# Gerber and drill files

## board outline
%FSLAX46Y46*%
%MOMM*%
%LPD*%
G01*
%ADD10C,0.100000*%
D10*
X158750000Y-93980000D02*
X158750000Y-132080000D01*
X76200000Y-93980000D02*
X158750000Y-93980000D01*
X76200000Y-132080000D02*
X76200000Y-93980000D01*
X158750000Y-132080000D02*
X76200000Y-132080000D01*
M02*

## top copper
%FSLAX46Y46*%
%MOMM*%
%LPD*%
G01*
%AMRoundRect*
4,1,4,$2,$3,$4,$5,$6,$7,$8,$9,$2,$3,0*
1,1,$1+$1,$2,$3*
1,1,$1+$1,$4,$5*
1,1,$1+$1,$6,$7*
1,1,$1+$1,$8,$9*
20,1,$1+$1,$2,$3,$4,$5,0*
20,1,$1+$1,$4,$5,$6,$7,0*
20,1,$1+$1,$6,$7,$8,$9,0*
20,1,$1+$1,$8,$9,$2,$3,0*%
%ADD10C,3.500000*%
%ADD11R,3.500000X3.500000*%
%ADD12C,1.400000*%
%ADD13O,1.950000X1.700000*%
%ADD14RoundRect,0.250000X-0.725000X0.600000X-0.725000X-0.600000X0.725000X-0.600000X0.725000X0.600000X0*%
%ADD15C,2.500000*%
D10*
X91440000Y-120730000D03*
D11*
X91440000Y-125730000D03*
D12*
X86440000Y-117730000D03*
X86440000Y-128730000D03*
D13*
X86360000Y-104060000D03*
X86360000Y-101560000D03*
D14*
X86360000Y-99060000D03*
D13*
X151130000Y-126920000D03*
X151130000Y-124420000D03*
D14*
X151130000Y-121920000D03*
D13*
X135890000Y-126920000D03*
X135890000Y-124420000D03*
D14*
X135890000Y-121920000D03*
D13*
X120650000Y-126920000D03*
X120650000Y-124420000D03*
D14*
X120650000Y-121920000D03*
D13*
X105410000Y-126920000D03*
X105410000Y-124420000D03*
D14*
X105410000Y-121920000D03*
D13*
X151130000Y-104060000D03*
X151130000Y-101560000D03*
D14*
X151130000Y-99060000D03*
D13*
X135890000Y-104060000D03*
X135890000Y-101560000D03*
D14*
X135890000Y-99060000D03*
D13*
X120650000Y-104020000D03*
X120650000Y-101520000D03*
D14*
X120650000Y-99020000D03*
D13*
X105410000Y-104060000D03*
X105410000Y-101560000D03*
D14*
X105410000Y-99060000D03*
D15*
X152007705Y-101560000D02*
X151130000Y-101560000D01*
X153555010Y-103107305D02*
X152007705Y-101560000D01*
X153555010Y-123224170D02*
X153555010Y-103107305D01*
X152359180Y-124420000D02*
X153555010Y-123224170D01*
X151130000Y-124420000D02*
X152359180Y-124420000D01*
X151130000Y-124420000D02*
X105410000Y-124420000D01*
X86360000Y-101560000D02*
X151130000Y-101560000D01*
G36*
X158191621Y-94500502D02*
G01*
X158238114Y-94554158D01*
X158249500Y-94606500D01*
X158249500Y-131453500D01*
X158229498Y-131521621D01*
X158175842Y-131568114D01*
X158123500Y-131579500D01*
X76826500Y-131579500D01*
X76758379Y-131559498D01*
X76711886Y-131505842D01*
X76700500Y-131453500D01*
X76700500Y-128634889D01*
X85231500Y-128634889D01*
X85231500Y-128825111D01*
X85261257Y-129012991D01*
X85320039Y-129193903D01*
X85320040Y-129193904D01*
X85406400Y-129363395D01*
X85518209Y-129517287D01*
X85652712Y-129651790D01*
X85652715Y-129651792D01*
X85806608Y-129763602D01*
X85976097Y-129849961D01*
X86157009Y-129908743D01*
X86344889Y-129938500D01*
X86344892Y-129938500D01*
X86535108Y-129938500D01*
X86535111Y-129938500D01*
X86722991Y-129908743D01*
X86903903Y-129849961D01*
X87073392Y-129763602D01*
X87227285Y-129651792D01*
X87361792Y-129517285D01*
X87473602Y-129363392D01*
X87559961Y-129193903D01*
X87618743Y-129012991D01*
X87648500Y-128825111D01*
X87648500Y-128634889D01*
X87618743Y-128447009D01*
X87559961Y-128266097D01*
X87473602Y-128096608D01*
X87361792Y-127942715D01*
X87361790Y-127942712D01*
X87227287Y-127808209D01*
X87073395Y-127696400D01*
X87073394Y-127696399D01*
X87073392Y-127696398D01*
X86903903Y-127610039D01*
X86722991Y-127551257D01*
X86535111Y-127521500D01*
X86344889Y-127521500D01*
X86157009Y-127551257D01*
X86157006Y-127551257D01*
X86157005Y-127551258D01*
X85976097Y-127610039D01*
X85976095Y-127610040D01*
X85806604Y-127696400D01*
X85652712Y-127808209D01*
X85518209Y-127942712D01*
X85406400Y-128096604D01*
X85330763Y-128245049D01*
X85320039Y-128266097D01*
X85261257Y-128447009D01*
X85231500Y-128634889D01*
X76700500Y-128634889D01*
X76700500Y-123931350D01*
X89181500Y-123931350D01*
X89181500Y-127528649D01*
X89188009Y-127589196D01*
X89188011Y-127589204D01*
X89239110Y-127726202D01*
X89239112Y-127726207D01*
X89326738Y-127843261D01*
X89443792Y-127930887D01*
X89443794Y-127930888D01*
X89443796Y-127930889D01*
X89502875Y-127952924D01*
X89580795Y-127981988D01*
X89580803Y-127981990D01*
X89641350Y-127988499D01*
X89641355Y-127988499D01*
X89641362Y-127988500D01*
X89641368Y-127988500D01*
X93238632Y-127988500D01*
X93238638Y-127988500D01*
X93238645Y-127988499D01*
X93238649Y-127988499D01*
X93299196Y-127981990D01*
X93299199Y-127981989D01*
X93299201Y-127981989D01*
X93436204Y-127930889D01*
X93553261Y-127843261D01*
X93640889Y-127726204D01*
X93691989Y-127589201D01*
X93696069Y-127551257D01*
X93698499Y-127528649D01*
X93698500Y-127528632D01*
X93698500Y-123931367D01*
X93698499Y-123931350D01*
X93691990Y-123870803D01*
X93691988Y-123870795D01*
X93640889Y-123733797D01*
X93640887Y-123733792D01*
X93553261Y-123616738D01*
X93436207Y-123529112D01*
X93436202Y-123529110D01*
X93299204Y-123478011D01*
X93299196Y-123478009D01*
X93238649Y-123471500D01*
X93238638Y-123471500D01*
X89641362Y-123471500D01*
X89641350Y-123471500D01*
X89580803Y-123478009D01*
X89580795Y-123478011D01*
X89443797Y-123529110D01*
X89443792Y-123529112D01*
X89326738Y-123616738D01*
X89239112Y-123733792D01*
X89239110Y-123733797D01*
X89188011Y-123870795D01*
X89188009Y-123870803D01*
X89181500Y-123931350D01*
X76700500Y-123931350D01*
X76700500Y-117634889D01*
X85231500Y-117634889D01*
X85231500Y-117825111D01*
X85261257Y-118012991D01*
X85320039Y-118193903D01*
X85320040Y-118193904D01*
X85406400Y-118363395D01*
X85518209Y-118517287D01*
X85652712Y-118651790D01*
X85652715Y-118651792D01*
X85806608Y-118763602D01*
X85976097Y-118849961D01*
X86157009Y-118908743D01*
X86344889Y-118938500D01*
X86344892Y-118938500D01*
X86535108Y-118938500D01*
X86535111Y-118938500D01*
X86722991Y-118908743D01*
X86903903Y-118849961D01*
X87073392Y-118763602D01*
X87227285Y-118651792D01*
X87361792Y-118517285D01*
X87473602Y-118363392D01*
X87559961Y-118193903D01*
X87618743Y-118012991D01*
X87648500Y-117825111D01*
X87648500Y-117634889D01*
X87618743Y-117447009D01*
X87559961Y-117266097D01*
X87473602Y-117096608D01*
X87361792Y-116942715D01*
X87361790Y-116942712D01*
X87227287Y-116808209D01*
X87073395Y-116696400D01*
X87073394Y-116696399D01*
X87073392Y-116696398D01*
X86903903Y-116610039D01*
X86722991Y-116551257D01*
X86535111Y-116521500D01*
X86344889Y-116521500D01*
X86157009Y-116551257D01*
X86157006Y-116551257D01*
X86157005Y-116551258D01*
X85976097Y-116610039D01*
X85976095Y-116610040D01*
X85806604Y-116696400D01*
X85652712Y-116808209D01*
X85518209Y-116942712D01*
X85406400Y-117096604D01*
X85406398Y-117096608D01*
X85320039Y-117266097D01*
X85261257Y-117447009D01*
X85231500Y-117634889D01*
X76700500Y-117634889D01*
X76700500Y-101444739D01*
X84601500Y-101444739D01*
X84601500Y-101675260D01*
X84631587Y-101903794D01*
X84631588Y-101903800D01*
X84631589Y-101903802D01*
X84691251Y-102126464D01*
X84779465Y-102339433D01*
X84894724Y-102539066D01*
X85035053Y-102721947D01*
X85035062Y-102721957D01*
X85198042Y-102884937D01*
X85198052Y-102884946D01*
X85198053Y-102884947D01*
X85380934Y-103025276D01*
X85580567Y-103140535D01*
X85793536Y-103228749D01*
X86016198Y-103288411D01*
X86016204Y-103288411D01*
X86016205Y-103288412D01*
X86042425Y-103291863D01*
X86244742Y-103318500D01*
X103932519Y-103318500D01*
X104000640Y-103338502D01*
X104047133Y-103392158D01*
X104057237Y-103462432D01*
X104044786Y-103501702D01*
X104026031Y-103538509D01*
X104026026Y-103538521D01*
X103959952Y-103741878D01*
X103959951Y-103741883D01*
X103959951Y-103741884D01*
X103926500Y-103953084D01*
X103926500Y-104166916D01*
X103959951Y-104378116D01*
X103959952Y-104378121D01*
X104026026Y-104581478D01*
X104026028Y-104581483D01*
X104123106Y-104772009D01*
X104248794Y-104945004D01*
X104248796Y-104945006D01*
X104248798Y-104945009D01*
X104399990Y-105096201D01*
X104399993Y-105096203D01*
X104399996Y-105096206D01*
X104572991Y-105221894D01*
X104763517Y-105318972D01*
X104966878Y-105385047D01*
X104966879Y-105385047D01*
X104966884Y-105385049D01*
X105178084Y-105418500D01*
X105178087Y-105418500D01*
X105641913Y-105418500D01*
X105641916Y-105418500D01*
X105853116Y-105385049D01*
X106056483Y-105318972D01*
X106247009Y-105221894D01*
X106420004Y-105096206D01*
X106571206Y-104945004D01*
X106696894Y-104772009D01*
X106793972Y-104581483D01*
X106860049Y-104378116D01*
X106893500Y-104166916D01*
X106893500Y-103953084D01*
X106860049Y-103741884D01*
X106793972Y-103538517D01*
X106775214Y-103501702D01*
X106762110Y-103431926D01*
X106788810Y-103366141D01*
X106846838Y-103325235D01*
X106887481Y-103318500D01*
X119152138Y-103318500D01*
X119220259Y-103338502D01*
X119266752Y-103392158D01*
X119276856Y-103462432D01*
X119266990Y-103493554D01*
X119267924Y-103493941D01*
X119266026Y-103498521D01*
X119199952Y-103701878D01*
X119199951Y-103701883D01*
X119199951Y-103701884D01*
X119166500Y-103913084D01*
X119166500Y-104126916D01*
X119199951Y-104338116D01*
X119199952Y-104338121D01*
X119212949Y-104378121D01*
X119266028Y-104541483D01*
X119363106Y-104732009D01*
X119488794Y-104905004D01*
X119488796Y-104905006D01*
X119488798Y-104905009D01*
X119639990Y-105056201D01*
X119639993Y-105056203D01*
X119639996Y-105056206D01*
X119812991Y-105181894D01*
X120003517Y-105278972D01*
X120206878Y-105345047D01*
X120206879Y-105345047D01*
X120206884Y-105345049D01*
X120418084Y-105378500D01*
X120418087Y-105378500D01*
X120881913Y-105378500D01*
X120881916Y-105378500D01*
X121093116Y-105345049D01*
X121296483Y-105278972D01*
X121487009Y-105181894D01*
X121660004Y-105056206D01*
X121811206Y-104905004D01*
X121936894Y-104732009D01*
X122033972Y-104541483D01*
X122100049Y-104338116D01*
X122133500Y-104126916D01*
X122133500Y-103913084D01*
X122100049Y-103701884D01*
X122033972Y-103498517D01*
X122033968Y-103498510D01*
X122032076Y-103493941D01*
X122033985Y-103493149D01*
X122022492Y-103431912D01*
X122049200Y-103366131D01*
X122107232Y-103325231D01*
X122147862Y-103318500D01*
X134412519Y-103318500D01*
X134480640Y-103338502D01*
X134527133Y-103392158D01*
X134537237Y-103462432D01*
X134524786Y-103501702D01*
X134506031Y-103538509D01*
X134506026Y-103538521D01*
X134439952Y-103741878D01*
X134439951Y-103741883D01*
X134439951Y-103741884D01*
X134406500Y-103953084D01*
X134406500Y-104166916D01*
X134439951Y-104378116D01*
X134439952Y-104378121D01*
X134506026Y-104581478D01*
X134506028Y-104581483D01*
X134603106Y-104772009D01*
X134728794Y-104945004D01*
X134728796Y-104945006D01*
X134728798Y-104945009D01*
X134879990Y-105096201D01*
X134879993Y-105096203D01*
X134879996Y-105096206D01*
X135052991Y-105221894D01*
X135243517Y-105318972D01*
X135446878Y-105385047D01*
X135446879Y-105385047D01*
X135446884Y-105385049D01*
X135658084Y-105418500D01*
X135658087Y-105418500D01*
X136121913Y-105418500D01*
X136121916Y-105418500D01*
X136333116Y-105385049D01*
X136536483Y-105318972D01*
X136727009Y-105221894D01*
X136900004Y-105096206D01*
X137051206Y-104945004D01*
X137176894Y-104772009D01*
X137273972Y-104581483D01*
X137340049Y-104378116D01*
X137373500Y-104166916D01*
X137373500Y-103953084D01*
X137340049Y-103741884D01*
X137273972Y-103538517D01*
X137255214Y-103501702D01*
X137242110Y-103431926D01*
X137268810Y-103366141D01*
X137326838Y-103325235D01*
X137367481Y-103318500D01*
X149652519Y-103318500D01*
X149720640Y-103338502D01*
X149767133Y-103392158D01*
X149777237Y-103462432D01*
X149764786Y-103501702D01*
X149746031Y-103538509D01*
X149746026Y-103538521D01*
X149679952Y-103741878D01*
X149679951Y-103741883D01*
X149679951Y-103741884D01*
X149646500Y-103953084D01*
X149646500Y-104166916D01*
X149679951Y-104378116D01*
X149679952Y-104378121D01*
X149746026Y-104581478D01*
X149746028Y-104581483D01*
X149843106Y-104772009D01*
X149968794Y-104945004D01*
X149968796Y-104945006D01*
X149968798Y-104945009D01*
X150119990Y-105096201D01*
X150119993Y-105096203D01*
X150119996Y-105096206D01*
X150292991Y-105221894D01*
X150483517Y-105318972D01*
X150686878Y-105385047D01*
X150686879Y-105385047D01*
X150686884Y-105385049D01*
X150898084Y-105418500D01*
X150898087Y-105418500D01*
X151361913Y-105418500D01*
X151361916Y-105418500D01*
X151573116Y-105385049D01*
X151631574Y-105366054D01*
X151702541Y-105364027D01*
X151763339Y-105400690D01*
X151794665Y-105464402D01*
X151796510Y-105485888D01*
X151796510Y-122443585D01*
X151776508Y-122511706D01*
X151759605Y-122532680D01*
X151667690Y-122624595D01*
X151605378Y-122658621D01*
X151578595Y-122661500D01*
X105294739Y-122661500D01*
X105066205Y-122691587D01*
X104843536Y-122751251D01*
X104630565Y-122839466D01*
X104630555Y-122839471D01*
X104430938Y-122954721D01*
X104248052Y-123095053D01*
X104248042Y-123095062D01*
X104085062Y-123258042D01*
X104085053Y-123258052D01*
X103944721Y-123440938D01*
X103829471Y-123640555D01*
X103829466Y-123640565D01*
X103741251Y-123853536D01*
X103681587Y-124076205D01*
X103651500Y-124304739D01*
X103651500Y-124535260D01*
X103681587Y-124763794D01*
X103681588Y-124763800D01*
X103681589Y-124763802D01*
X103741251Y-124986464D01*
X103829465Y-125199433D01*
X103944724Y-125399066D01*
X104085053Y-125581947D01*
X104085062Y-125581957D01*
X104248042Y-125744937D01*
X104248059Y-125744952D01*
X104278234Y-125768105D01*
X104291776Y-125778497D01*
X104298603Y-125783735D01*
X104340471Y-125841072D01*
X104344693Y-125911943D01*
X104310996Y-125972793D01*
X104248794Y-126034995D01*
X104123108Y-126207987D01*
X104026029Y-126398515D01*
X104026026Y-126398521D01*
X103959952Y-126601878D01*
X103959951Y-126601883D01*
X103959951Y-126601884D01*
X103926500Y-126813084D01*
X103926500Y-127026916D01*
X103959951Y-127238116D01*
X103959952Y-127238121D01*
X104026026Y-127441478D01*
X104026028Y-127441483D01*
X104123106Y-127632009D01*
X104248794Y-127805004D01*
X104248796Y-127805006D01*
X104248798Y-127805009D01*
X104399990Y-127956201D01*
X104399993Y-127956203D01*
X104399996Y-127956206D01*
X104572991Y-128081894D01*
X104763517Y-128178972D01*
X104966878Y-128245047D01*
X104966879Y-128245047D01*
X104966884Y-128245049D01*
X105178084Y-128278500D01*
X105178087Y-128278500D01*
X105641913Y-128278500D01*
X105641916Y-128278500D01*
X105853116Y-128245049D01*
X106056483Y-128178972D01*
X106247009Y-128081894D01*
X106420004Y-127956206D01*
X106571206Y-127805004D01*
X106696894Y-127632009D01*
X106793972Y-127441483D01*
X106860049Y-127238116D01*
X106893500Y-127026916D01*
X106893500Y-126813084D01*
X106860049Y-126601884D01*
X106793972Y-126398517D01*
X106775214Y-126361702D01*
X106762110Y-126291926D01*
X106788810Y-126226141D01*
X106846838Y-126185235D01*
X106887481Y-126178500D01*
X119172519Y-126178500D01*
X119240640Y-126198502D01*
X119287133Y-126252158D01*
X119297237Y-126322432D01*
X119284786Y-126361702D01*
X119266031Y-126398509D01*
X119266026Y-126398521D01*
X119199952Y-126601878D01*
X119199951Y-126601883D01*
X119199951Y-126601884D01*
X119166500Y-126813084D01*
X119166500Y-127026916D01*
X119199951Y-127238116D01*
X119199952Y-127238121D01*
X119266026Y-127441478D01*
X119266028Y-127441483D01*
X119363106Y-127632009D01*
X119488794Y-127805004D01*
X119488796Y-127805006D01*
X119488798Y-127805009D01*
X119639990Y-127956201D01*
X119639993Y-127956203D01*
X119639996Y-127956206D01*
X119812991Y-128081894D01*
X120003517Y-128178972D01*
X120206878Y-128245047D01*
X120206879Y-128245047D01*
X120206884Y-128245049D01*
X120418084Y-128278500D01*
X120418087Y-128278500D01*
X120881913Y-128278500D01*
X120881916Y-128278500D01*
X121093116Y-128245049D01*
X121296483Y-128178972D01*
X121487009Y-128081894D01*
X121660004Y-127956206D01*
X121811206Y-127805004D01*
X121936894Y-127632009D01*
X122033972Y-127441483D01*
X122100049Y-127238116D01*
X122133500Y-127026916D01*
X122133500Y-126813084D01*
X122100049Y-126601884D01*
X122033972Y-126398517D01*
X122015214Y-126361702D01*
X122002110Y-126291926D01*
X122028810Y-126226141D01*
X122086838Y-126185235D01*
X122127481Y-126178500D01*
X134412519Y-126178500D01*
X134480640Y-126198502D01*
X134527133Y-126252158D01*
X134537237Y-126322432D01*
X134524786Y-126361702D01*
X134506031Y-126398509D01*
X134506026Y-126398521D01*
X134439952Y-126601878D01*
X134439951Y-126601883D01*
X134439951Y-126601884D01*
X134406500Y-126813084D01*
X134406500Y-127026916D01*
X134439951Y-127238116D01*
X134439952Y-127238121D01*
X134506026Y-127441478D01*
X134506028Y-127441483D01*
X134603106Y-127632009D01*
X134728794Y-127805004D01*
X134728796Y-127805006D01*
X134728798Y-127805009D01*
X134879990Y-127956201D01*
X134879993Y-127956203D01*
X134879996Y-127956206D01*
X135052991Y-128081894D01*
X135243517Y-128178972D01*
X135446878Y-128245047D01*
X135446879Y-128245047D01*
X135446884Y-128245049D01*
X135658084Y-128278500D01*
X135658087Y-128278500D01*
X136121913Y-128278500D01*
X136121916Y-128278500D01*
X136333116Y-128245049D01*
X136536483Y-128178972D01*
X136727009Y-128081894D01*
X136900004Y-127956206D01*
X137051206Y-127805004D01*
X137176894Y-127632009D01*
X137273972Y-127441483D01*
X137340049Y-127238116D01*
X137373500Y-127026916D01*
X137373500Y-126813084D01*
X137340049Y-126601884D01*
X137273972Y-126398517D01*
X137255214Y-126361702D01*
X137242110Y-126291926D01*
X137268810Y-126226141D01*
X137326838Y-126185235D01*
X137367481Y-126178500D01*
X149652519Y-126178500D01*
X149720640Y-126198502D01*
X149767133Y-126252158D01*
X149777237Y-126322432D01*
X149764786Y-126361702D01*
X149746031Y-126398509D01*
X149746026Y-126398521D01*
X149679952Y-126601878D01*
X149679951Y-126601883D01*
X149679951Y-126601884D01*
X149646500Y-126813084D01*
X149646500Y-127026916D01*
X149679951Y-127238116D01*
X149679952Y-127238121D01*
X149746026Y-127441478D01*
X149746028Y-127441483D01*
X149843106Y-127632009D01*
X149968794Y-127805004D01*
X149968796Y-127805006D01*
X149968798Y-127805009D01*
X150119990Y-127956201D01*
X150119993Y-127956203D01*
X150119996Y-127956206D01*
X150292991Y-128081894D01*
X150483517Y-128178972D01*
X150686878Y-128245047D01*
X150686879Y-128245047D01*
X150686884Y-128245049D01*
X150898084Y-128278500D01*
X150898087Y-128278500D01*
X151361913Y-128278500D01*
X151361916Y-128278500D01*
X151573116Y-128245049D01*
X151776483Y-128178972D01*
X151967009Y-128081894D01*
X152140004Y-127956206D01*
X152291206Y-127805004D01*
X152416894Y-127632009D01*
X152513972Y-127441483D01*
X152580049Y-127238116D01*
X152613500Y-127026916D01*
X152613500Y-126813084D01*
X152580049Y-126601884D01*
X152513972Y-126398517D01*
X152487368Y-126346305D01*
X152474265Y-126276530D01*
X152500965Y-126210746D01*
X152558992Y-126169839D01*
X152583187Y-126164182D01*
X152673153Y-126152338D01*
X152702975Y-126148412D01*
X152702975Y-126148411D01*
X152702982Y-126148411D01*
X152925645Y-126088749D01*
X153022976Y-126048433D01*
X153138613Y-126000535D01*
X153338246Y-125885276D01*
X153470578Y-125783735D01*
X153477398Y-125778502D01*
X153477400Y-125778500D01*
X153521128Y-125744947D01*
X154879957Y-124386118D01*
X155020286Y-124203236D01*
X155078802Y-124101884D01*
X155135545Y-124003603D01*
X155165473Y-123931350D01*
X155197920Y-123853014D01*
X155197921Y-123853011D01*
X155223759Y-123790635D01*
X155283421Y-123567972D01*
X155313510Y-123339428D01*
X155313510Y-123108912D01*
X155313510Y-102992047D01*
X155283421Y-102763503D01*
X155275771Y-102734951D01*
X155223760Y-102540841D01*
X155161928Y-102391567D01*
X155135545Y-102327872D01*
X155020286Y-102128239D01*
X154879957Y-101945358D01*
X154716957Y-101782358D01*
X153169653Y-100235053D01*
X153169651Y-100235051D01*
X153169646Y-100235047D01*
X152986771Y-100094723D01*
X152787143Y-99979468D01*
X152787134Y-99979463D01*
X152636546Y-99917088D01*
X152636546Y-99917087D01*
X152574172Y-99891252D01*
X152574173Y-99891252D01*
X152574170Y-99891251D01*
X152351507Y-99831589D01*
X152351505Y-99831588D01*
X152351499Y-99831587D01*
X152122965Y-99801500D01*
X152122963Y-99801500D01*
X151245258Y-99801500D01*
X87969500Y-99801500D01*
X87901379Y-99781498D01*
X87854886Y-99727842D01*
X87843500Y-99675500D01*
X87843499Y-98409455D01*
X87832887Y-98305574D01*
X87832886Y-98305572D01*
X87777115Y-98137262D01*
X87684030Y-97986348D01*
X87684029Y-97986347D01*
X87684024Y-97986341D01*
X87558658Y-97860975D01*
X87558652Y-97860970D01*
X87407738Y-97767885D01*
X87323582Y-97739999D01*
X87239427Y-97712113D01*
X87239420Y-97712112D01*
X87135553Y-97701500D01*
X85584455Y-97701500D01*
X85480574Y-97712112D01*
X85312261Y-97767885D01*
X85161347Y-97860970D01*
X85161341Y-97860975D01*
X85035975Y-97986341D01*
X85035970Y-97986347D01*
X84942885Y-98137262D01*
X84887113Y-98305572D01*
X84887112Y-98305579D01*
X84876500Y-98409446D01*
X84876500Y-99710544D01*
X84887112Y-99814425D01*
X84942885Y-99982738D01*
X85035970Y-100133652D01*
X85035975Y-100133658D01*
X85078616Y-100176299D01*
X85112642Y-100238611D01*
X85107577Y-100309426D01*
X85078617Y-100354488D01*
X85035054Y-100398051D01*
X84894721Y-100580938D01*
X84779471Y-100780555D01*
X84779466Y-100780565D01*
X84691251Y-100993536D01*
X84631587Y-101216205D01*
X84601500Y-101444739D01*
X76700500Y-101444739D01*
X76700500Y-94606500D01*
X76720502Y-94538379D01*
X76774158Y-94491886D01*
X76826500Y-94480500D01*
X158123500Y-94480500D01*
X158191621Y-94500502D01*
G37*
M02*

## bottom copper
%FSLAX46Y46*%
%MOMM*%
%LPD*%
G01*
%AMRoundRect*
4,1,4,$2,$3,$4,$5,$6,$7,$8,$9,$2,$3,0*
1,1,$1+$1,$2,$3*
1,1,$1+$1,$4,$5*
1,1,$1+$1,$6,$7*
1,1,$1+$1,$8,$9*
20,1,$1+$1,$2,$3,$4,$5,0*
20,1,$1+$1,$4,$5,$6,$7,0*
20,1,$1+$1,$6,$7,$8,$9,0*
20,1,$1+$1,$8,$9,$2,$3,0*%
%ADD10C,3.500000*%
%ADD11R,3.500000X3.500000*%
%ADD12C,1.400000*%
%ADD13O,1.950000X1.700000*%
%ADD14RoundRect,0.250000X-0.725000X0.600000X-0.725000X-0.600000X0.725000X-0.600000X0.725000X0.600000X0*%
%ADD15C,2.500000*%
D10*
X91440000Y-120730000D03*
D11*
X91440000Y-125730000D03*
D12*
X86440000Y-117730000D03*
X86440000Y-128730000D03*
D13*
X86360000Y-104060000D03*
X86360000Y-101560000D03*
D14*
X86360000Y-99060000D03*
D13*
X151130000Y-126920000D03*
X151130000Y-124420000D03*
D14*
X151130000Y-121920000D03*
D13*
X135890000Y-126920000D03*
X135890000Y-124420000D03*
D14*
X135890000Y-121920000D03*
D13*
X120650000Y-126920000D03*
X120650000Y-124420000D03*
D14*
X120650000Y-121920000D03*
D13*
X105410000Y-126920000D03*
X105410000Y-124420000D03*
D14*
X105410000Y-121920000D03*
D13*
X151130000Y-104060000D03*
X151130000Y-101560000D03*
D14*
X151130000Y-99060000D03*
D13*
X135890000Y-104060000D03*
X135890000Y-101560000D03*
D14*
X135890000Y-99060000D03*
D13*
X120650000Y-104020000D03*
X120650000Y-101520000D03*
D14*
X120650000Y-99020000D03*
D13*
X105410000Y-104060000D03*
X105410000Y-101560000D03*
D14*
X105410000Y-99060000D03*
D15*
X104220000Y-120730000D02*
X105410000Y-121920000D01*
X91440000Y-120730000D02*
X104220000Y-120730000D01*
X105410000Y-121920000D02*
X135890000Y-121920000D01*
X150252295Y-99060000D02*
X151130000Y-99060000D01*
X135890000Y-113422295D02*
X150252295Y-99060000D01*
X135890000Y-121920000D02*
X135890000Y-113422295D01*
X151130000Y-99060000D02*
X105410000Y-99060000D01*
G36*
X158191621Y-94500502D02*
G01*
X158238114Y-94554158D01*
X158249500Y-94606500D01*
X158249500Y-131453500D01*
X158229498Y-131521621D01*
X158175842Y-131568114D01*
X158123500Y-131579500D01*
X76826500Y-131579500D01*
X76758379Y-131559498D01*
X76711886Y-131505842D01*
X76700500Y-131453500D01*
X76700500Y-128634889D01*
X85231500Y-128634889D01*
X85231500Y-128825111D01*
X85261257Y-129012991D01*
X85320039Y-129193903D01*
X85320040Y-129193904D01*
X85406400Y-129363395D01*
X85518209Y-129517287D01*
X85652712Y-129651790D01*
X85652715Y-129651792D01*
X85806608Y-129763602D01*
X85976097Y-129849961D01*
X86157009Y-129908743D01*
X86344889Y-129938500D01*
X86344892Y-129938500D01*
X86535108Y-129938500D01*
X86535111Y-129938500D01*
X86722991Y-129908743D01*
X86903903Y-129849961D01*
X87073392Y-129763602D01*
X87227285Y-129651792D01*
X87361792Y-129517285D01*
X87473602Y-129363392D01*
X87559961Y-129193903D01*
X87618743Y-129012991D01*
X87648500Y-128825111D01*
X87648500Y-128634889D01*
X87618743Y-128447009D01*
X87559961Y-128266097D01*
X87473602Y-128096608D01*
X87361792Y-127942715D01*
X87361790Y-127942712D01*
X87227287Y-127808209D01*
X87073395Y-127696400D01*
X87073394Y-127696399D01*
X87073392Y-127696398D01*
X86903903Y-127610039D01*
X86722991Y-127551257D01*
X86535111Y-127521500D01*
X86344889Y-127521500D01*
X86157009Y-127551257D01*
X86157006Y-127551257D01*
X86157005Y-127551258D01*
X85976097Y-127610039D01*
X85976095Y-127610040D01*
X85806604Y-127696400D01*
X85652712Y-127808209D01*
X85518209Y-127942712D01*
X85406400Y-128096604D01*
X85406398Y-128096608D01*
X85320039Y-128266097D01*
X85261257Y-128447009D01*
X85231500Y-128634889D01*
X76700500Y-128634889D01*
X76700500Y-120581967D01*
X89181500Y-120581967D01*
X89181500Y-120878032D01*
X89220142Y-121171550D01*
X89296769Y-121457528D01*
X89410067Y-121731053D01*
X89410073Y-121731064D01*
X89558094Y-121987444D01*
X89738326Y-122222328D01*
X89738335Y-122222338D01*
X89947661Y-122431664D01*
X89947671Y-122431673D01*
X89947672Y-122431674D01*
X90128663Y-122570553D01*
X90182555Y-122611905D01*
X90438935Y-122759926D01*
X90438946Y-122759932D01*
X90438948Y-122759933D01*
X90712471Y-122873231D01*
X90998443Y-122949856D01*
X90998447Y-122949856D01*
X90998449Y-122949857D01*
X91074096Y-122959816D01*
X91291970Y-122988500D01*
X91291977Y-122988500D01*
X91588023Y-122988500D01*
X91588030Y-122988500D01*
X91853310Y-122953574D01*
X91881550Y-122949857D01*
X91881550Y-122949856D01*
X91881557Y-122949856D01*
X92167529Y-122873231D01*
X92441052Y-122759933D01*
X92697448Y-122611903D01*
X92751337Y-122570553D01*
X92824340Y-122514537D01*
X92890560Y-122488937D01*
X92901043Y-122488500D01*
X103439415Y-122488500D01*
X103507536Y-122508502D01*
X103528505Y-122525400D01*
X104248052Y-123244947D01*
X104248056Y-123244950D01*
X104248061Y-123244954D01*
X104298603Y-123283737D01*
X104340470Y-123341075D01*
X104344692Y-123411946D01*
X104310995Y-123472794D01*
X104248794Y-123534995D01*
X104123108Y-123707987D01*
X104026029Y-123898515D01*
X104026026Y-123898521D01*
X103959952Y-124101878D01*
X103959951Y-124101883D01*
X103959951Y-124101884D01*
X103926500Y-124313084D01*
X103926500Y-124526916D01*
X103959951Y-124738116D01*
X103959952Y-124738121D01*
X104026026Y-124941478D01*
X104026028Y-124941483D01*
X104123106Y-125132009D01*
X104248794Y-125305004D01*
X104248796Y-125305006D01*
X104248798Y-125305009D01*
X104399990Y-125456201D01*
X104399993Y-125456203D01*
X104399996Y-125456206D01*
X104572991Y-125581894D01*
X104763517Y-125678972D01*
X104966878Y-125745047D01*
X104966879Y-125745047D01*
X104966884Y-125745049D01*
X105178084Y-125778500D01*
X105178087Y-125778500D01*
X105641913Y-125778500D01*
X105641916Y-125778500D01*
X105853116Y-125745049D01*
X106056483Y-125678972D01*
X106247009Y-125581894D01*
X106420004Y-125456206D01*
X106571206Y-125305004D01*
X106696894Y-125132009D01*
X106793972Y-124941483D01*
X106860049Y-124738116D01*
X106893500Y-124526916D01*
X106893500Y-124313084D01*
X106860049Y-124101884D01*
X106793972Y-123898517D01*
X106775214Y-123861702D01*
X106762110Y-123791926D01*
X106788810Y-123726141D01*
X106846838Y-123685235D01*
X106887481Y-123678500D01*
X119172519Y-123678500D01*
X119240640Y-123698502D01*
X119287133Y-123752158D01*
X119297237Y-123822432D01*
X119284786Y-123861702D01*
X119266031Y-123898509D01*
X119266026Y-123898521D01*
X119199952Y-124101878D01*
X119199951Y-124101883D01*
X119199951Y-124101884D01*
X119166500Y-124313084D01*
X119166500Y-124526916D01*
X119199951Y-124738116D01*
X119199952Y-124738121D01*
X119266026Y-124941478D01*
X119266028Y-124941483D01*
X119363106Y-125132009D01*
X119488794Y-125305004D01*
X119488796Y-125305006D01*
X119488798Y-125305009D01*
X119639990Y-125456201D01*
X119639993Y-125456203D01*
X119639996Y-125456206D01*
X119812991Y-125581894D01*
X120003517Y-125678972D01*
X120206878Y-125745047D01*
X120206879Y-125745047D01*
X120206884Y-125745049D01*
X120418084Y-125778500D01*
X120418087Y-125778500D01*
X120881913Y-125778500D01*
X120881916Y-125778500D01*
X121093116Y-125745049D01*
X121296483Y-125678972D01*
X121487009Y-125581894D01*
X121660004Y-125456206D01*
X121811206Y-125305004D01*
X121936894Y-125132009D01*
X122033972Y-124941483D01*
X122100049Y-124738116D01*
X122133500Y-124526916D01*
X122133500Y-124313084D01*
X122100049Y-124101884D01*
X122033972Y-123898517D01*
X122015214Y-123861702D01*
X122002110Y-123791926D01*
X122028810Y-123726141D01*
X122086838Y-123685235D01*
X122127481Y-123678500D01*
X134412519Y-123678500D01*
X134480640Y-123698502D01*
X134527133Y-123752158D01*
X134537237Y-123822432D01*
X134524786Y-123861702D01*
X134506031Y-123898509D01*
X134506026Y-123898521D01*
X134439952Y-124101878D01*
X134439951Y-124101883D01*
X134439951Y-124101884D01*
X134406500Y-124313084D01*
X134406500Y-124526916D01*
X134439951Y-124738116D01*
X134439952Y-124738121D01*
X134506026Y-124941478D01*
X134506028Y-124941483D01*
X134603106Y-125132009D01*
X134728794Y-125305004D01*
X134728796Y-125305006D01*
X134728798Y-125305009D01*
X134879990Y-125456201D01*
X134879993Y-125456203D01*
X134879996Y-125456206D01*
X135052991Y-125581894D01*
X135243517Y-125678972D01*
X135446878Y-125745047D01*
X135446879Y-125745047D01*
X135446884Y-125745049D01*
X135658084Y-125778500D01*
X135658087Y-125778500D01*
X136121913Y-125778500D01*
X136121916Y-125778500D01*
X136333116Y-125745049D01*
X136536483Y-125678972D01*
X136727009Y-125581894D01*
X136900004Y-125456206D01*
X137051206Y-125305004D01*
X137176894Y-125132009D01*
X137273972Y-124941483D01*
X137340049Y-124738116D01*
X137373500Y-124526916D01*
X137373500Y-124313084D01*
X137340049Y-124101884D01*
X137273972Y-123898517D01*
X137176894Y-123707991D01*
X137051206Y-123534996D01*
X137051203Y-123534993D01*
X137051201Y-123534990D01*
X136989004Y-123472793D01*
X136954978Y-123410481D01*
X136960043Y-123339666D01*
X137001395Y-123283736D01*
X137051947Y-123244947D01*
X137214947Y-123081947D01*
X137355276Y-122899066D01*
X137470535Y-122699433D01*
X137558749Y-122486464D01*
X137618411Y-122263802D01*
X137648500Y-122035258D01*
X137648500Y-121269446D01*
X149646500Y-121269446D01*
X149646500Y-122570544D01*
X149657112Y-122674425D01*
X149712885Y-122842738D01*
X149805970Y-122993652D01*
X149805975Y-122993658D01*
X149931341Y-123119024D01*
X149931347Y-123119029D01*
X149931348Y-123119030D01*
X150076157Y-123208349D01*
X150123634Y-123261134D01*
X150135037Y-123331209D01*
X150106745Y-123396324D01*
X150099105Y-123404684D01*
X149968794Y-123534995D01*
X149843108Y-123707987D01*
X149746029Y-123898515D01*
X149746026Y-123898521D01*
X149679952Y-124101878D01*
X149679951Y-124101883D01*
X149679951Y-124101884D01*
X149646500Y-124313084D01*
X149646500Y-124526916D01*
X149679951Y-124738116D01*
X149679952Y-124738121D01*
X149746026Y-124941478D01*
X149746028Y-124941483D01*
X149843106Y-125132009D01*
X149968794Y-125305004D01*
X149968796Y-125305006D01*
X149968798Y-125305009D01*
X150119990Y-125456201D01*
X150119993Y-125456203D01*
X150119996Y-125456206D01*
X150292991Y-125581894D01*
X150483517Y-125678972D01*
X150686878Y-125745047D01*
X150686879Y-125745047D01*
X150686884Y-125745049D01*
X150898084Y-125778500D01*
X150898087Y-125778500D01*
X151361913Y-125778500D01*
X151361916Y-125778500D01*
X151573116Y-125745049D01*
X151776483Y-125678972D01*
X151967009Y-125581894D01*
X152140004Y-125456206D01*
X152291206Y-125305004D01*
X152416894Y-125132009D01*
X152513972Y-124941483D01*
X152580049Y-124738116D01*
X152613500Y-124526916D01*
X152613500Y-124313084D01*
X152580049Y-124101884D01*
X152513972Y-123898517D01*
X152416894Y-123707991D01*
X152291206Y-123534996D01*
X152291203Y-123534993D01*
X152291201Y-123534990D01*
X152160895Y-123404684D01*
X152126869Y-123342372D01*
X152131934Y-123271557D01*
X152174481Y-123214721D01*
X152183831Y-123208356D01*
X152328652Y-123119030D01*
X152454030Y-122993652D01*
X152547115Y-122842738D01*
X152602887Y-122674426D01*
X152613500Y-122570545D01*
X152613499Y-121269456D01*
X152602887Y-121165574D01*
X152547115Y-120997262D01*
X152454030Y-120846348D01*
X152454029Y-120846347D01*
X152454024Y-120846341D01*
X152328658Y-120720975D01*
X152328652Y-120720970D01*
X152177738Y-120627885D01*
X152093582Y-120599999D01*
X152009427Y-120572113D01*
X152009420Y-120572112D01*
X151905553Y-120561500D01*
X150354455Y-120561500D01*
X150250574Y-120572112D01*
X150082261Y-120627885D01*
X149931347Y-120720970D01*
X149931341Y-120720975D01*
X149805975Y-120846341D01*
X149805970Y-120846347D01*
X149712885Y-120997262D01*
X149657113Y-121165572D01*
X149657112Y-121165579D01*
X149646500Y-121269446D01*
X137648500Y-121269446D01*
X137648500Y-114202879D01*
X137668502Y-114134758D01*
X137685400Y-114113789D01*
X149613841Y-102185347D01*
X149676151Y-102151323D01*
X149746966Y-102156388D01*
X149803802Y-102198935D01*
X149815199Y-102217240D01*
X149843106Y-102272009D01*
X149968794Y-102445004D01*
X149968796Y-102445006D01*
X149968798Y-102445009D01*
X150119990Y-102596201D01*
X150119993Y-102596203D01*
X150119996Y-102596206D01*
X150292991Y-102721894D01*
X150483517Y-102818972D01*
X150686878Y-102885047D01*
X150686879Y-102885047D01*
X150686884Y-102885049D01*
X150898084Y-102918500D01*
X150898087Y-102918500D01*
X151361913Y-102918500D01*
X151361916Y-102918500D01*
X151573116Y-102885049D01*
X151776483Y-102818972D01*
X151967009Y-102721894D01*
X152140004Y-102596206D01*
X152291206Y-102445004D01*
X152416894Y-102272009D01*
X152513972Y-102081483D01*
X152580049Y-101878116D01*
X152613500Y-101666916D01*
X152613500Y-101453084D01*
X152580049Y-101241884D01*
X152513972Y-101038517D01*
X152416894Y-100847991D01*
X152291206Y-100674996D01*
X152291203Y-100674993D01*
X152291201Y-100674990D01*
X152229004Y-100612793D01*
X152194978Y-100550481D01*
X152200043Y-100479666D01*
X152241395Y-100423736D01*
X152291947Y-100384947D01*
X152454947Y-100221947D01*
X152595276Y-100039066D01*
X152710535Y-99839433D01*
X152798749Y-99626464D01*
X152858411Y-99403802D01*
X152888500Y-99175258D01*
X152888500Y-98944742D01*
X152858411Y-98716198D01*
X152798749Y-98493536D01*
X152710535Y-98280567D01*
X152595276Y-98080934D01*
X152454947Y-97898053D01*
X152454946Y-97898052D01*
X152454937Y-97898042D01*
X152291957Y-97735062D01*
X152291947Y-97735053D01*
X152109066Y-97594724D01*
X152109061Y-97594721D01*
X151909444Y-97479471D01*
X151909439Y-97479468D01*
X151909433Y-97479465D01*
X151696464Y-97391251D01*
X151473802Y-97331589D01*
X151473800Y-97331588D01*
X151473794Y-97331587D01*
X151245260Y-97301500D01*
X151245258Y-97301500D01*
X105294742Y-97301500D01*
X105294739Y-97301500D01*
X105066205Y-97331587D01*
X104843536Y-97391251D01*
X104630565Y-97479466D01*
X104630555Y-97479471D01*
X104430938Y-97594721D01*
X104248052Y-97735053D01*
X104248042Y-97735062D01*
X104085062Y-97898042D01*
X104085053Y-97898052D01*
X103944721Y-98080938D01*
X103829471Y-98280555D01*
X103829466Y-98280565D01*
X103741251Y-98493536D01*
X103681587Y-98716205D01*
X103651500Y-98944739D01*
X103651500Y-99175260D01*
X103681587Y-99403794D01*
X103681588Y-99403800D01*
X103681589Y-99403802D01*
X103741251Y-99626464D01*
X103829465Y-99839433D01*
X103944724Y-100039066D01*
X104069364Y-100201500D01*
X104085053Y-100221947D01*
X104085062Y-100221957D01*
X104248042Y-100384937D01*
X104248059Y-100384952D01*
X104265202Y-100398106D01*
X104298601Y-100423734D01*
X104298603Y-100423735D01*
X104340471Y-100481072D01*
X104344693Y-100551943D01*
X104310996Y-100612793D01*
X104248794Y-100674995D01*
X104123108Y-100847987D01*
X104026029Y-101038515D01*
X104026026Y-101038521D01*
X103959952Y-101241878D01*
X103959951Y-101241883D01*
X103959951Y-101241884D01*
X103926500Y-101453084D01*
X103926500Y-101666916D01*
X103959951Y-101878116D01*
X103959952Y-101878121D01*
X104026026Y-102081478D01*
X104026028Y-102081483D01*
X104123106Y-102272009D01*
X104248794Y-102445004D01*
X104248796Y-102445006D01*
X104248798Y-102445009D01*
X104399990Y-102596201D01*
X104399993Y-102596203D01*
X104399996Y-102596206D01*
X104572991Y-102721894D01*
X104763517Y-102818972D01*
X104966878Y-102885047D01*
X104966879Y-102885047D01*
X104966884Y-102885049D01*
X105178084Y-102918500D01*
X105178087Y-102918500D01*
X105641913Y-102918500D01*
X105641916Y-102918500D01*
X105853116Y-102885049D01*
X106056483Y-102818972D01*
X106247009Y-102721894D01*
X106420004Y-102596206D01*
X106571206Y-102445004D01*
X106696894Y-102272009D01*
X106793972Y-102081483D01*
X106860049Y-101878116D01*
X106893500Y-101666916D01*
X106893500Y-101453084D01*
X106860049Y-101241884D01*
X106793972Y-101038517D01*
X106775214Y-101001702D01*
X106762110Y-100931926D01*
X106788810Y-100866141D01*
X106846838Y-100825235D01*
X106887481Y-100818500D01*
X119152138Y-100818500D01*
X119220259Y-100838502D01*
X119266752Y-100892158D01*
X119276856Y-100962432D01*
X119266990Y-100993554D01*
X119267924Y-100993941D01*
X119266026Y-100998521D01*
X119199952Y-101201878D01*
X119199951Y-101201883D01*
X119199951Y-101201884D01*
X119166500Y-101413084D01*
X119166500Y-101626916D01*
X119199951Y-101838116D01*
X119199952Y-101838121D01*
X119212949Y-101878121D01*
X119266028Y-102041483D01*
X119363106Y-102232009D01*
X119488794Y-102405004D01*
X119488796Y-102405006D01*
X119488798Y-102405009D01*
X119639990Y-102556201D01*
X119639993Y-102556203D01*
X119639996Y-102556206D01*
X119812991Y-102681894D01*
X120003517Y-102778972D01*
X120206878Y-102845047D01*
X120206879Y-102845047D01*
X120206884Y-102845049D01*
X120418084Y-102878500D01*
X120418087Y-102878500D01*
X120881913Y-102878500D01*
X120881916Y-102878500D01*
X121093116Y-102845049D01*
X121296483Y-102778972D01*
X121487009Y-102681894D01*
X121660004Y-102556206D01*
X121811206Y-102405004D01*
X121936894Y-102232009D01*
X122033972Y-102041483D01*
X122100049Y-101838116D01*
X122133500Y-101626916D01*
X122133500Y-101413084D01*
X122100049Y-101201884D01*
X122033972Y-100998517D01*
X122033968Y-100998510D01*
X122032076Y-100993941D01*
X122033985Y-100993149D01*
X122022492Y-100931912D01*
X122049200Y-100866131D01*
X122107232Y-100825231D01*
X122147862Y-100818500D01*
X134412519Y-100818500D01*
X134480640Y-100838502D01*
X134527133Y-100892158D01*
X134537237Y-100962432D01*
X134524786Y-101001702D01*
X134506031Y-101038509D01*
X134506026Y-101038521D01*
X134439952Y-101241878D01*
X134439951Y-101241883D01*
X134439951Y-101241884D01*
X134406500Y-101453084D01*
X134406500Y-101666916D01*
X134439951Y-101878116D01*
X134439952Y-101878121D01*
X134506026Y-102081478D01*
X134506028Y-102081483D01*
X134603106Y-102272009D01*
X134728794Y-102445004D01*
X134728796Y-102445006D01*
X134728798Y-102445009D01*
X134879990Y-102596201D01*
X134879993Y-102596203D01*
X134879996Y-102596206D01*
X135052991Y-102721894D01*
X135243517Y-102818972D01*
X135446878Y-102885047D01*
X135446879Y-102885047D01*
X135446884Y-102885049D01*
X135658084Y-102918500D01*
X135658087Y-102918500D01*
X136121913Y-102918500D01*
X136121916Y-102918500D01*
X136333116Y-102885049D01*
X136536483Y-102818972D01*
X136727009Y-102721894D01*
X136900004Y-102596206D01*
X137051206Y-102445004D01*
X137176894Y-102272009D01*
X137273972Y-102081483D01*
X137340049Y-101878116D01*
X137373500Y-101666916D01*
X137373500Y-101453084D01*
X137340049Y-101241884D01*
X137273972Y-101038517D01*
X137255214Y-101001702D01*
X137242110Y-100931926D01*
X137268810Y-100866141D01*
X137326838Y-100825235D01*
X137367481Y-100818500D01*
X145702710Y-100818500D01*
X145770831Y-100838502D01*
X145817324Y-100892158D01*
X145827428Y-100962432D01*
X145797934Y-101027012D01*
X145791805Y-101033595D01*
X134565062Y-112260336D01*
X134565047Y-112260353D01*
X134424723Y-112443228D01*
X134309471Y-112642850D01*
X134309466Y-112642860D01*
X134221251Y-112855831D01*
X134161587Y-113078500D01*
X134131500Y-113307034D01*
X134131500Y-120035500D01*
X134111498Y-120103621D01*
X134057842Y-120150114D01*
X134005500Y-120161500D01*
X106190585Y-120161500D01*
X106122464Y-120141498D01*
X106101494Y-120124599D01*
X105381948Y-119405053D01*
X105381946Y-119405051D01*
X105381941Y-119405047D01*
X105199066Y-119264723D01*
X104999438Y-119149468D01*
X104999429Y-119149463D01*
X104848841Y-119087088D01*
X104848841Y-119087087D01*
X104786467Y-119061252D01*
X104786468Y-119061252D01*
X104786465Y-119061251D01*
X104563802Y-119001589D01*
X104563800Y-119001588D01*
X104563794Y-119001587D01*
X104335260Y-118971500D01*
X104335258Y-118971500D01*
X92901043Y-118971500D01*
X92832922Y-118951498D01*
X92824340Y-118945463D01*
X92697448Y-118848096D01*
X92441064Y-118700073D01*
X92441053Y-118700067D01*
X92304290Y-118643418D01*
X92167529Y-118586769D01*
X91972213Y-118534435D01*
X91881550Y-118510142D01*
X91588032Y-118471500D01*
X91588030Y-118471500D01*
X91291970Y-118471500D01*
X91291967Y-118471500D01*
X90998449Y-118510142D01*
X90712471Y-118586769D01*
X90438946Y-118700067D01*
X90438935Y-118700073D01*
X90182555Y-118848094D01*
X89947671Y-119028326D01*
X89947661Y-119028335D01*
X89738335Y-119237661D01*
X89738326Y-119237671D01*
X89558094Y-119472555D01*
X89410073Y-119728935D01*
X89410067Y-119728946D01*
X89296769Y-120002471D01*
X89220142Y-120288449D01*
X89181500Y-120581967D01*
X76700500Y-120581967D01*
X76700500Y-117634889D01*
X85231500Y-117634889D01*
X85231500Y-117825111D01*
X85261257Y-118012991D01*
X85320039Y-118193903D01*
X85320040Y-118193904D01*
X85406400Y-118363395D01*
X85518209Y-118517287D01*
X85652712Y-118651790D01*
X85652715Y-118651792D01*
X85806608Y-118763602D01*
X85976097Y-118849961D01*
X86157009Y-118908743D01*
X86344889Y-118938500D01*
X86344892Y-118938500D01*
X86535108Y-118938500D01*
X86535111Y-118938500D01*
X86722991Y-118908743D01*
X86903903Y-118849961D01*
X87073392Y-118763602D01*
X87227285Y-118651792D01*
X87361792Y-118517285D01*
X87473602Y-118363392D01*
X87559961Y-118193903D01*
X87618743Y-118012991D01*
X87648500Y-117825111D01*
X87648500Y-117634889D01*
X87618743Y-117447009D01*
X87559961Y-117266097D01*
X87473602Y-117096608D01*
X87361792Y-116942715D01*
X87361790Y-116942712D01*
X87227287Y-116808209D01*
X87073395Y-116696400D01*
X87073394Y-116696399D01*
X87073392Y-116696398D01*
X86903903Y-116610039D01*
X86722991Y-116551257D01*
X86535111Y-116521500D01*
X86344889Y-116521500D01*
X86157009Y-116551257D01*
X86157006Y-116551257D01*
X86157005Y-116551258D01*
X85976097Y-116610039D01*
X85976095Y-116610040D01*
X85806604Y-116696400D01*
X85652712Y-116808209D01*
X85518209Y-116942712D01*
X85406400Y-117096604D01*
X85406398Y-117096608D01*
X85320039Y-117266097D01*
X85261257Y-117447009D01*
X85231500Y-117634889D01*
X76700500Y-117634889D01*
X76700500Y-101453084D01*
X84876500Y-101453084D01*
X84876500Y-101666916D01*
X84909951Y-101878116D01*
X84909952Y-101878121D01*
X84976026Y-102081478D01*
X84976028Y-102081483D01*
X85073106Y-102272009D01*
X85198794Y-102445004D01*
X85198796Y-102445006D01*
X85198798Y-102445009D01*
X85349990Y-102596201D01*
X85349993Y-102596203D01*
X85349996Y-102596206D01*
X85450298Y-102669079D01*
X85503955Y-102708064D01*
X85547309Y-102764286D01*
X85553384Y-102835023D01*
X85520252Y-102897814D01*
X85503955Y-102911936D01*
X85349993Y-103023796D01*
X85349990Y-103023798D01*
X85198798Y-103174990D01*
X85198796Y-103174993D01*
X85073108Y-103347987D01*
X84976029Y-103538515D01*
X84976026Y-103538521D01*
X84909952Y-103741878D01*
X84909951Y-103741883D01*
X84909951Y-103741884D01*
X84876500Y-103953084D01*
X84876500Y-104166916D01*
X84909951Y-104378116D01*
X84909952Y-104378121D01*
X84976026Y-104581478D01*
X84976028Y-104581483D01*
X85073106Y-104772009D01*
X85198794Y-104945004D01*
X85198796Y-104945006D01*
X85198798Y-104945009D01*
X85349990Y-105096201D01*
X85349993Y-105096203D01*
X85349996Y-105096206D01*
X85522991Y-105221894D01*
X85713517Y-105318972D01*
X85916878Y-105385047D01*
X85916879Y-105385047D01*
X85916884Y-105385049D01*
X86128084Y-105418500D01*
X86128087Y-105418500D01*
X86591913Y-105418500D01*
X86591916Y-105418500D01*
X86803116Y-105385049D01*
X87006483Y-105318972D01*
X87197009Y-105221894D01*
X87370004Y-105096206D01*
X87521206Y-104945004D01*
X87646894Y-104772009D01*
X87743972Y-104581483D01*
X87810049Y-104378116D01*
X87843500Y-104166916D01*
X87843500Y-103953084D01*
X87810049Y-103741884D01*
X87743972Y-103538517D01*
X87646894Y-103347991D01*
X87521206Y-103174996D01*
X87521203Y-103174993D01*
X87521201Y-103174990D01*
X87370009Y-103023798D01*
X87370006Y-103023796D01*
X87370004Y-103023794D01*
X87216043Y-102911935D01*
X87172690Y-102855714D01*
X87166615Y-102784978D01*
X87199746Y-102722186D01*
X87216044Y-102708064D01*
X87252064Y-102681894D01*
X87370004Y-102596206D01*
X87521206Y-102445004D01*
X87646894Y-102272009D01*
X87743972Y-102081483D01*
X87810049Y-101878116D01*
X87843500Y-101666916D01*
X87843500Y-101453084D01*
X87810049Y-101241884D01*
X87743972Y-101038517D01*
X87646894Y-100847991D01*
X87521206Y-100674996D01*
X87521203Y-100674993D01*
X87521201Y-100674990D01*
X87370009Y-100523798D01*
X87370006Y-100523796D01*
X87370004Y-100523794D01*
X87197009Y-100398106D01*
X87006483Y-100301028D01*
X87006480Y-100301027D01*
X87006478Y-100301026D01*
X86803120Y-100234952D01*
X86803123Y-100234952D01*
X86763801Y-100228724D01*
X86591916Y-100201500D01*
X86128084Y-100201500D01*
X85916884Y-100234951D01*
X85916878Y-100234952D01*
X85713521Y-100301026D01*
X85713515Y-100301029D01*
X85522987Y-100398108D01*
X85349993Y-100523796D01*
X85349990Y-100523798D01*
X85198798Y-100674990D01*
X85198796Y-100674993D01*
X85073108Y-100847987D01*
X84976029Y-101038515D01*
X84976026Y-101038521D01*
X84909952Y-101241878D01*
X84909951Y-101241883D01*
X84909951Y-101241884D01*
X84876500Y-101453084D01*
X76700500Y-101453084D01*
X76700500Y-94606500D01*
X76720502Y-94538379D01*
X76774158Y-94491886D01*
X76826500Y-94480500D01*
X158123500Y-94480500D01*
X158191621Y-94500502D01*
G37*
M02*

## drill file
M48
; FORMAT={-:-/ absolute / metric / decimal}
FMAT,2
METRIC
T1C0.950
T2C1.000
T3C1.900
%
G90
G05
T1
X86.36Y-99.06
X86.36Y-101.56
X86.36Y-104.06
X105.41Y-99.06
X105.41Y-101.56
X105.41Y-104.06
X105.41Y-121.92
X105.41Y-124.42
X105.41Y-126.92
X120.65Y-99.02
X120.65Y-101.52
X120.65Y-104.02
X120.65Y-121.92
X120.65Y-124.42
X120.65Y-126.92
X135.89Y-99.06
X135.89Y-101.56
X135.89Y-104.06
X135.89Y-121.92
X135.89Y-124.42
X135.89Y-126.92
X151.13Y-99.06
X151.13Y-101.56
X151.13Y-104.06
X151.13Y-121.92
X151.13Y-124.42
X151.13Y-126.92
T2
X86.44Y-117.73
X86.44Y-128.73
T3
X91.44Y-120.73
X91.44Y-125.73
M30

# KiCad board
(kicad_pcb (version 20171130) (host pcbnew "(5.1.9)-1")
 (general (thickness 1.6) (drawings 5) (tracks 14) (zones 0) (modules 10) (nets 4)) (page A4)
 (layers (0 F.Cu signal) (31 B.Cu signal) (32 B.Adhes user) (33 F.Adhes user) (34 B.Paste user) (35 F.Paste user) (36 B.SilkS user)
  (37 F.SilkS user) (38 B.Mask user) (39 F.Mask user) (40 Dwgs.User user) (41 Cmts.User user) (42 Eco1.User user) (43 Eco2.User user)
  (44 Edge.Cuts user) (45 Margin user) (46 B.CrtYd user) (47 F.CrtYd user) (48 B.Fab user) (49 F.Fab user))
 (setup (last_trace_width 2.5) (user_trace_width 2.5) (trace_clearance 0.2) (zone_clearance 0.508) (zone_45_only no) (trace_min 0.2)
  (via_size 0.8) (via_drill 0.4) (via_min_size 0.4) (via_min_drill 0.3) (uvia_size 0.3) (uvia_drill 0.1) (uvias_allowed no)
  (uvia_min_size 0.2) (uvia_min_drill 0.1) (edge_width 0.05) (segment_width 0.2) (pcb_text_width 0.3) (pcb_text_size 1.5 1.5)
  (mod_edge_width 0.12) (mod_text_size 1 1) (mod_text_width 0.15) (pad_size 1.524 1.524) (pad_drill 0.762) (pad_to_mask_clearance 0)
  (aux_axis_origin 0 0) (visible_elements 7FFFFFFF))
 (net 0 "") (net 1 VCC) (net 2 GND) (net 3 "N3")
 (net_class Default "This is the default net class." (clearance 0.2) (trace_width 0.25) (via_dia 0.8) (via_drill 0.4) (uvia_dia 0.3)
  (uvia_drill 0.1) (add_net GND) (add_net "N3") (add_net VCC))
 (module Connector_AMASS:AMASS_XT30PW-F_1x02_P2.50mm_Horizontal (layer F.Cu) (at 91.44 125.73 90)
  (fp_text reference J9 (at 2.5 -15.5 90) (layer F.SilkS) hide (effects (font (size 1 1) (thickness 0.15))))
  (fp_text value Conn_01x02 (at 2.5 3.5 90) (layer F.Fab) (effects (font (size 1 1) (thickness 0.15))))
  (pad 2 thru_hole circle (at 5 0 90) (size 3.5 3.5) (drill 1.9) (layers *.Cu *.Mask) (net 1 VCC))
  (pad 1 thru_hole rect (at 0 0 90) (size 3.5 3.5) (drill 1.9) (layers *.Cu *.Mask) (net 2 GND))
  (pad "" thru_hole circle (at 8 -5 90) (size 1.4 1.4) (drill 1) (layers *.Cu *.Mask))
  (pad "" thru_hole circle (at -3 -5 180) (size 1.4 1.4) (drill 1) (layers *.Cu *.Mask)))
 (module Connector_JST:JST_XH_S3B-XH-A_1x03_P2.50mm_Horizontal (layer F.Cu) (at 86.36 99.06 270)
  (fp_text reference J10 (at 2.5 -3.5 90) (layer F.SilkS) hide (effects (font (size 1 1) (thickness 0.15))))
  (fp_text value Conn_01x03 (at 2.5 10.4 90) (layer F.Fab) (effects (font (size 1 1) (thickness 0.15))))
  (pad 3 thru_hole oval (at 5 0 270) (size 1.7 1.95) (drill 0.95) (layers *.Cu *.Mask) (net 1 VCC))
  (pad 2 thru_hole oval (at 2.5 0 270) (size 1.7 1.95) (drill 0.95) (layers *.Cu *.Mask) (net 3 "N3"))
  (pad 1 thru_hole roundrect (at 0 0 270) (size 1.7 1.95) (drill 0.95) (layers *.Cu *.Mask) (roundrect_rratio 0.1470588235294118)
   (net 2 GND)))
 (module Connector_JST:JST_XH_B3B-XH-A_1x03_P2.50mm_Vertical (layer F.Cu) (at 151.13 121.92 270)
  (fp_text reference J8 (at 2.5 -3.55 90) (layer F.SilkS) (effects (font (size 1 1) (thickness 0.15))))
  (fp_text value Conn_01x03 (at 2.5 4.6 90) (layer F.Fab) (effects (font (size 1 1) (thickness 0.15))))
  (pad 3 thru_hole oval (at 5 0 270) (size 1.7 1.95) (drill 0.95) (layers *.Cu *.Mask) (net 2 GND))
  (pad 2 thru_hole oval (at 2.5 0 270) (size 1.7 1.95) (drill 0.95) (layers *.Cu *.Mask) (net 3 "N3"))
  (pad 1 thru_hole roundrect (at 0 0 270) (size 1.7 1.95) (drill 0.95) (layers *.Cu *.Mask) (roundrect_rratio 0.1470588235294118)
   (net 1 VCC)))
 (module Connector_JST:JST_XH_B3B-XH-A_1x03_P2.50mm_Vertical (layer F.Cu) (at 135.89 121.92 270)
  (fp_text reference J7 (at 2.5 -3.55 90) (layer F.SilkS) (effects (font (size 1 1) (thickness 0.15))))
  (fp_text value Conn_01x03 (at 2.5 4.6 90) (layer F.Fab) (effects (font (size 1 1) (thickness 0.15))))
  (pad 3 thru_hole oval (at 5 0 270) (size 1.7 1.95) (drill 0.95) (layers *.Cu *.Mask) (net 2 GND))
  (pad 2 thru_hole oval (at 2.5 0 270) (size 1.7 1.95) (drill 0.95) (layers *.Cu *.Mask) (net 3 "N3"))
  (pad 1 thru_hole roundrect (at 0 0 270) (size 1.7 1.95) (drill 0.95) (layers *.Cu *.Mask) (roundrect_rratio 0.1470588235294118)
   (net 1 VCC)))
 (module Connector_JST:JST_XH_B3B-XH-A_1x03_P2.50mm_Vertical (layer F.Cu) (at 120.65 121.92 270)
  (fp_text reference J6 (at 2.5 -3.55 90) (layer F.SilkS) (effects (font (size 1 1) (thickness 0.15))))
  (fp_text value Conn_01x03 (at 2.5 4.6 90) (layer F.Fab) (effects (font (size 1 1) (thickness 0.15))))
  (pad 3 thru_hole oval (at 5 0 270) (size 1.7 1.95) (drill 0.95) (layers *.Cu *.Mask) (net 2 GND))
  (pad 2 thru_hole oval (at 2.5 0 270) (size 1.7 1.95) (drill 0.95) (layers *.Cu *.Mask) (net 3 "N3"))
  (pad 1 thru_hole roundrect (at 0 0 270) (size 1.7 1.95) (drill 0.95) (layers *.Cu *.Mask) (roundrect_rratio 0.1470588235294118)
   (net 1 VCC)))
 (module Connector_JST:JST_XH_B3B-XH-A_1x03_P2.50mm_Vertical (layer F.Cu) (at 105.41 121.92 270)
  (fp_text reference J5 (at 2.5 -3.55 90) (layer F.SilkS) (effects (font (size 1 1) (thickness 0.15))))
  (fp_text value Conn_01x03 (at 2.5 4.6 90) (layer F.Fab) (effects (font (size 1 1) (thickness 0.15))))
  (pad 3 thru_hole oval (at 5 0 270) (size 1.7 1.95) (drill 0.95) (layers *.Cu *.Mask) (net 2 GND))
  (pad 2 thru_hole oval (at 2.5 0 270) (size 1.7 1.95) (drill 0.95) (layers *.Cu *.Mask) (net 3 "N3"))
  (pad 1 thru_hole roundrect (at 0 0 270) (size 1.7 1.95) (drill 0.95) (layers *.Cu *.Mask) (roundrect_rratio 0.1470588235294118)
   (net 1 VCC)))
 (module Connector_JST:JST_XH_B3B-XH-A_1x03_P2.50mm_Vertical (layer F.Cu) (at 151.13 99.06 270)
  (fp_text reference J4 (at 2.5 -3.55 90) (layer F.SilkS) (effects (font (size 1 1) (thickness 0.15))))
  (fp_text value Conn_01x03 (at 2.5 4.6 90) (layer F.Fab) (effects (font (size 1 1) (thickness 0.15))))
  (pad 3 thru_hole oval (at 5 0 270) (size 1.7 1.95) (drill 0.95) (layers *.Cu *.Mask) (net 2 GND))
  (pad 2 thru_hole oval (at 2.5 0 270) (size 1.7 1.95) (drill 0.95) (layers *.Cu *.Mask) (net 3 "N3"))
  (pad 1 thru_hole roundrect (at 0 0 270) (size 1.7 1.95) (drill 0.95) (layers *.Cu *.Mask) (roundrect_rratio 0.1470588235294118)
   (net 1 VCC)))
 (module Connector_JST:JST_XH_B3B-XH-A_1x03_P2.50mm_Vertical (layer F.Cu) (at 135.89 99.06 270)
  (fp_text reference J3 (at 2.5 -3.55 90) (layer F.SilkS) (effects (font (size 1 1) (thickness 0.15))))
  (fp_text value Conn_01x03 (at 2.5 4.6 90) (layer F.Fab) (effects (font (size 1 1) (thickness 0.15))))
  (pad 3 thru_hole oval (at 5 0 270) (size 1.7 1.95) (drill 0.95) (layers *.Cu *.Mask) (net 2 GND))
  (pad 2 thru_hole oval (at 2.5 0 270) (size 1.7 1.95) (drill 0.95) (layers *.Cu *.Mask) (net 3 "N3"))
  (pad 1 thru_hole roundrect (at 0 0 270) (size 1.7 1.95) (drill 0.95) (layers *.Cu *.Mask) (roundrect_rratio 0.1470588235294118)
   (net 1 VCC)))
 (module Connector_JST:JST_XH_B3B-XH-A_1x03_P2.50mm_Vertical (layer F.Cu) (at 120.65 99.02 270)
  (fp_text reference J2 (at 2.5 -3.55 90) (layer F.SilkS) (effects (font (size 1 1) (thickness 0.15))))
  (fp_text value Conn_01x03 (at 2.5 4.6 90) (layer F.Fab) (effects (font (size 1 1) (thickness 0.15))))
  (pad 3 thru_hole oval (at 5 0 270) (size 1.7 1.95) (drill 0.95) (layers *.Cu *.Mask) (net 2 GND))
  (pad 2 thru_hole oval (at 2.5 0 270) (size 1.7 1.95) (drill 0.95) (layers *.Cu *.Mask) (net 3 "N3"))
  (pad 1 thru_hole roundrect (at 0 0 270) (size 1.7 1.95) (drill 0.95) (layers *.Cu *.Mask) (roundrect_rratio 0.1470588235294118)
   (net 1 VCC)))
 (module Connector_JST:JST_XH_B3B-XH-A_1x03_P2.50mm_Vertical (layer F.Cu) (at 105.41 99.06 270)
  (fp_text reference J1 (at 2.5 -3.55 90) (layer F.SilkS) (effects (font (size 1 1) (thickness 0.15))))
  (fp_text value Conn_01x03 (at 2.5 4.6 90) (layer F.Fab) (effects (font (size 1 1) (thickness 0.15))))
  (pad 3 thru_hole oval (at 5 0 270) (size 1.7 1.95) (drill 0.95) (layers *.Cu *.Mask) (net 2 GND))
  (pad 2 thru_hole oval (at 2.5 0 270) (size 1.7 1.95) (drill 0.95) (layers *.Cu *.Mask) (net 3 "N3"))
  (pad 1 thru_hole roundrect (at 0 0 270) (size 1.7 1.95) (drill 0.95) (layers *.Cu *.Mask) (roundrect_rratio 0.1470588235294118)
   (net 1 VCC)))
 (gr_line (start 158.75 93.98) (end 158.75 132.08) (layer Edge.Cuts) (width 0.1))
 (gr_line (start 76.2 93.98) (end 158.75 93.98) (layer Edge.Cuts) (width 0.1))
 (gr_line (start 76.2 132.08) (end 76.2 93.98) (layer Edge.Cuts) (width 0.1))
 (gr_line (start 158.75 132.08) (end 76.2 132.08) (layer Edge.Cuts) (width 0.1))
 (segment (start 104.22 120.73) (end 105.41 121.92) (width 2.5) (layer B.Cu) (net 1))
 (segment (start 91.44 120.73) (end 104.22 120.73) (width 2.5) (layer B.Cu) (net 1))
 (segment (start 105.41 121.92) (end 135.89 121.92) (width 2.5) (layer B.Cu) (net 1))
 (segment (start 150.252295 99.06) (end 151.13 99.06) (width 2.5) (layer B.Cu) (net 1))
 (segment (start 135.89 113.422295) (end 150.252295 99.06) (width 2.5) (layer B.Cu) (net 1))
 (segment (start 135.89 121.92) (end 135.89 113.422295) (width 2.5) (layer B.Cu) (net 1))
 (segment (start 151.13 99.06) (end 105.41 99.06) (width 2.5) (layer B.Cu) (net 1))
 (segment (start 152.007705 101.56) (end 151.13 101.56) (width 2.5) (layer F.Cu) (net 3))
 (segment (start 153.55501 103.107305) (end 152.007705 101.56) (width 2.5) (layer F.Cu) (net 3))
 (segment (start 153.55501 123.22417) (end 153.55501 103.107305) (width 2.5) (layer F.Cu) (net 3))
 (segment (start 152.35918 124.42) (end 153.55501 123.22417) (width 2.5) (layer F.Cu) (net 3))
 (segment (start 151.13 124.42) (end 152.35918 124.42) (width 2.5) (layer F.Cu) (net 3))
 (segment (start 151.13 124.42) (end 105.41 124.42) (width 2.5) (layer F.Cu) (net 3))
 (segment (start 86.36 101.56) (end 151.13 101.56) (width 2.5) (layer F.Cu) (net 3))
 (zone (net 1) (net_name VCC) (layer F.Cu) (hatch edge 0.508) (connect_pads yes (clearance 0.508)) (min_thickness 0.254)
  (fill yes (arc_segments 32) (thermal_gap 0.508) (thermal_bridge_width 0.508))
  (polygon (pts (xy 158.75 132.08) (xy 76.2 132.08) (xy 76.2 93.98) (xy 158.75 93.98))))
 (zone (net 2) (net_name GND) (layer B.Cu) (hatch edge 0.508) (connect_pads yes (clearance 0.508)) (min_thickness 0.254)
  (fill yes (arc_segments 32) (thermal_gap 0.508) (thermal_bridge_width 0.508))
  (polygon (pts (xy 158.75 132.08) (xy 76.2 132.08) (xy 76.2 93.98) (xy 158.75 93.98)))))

